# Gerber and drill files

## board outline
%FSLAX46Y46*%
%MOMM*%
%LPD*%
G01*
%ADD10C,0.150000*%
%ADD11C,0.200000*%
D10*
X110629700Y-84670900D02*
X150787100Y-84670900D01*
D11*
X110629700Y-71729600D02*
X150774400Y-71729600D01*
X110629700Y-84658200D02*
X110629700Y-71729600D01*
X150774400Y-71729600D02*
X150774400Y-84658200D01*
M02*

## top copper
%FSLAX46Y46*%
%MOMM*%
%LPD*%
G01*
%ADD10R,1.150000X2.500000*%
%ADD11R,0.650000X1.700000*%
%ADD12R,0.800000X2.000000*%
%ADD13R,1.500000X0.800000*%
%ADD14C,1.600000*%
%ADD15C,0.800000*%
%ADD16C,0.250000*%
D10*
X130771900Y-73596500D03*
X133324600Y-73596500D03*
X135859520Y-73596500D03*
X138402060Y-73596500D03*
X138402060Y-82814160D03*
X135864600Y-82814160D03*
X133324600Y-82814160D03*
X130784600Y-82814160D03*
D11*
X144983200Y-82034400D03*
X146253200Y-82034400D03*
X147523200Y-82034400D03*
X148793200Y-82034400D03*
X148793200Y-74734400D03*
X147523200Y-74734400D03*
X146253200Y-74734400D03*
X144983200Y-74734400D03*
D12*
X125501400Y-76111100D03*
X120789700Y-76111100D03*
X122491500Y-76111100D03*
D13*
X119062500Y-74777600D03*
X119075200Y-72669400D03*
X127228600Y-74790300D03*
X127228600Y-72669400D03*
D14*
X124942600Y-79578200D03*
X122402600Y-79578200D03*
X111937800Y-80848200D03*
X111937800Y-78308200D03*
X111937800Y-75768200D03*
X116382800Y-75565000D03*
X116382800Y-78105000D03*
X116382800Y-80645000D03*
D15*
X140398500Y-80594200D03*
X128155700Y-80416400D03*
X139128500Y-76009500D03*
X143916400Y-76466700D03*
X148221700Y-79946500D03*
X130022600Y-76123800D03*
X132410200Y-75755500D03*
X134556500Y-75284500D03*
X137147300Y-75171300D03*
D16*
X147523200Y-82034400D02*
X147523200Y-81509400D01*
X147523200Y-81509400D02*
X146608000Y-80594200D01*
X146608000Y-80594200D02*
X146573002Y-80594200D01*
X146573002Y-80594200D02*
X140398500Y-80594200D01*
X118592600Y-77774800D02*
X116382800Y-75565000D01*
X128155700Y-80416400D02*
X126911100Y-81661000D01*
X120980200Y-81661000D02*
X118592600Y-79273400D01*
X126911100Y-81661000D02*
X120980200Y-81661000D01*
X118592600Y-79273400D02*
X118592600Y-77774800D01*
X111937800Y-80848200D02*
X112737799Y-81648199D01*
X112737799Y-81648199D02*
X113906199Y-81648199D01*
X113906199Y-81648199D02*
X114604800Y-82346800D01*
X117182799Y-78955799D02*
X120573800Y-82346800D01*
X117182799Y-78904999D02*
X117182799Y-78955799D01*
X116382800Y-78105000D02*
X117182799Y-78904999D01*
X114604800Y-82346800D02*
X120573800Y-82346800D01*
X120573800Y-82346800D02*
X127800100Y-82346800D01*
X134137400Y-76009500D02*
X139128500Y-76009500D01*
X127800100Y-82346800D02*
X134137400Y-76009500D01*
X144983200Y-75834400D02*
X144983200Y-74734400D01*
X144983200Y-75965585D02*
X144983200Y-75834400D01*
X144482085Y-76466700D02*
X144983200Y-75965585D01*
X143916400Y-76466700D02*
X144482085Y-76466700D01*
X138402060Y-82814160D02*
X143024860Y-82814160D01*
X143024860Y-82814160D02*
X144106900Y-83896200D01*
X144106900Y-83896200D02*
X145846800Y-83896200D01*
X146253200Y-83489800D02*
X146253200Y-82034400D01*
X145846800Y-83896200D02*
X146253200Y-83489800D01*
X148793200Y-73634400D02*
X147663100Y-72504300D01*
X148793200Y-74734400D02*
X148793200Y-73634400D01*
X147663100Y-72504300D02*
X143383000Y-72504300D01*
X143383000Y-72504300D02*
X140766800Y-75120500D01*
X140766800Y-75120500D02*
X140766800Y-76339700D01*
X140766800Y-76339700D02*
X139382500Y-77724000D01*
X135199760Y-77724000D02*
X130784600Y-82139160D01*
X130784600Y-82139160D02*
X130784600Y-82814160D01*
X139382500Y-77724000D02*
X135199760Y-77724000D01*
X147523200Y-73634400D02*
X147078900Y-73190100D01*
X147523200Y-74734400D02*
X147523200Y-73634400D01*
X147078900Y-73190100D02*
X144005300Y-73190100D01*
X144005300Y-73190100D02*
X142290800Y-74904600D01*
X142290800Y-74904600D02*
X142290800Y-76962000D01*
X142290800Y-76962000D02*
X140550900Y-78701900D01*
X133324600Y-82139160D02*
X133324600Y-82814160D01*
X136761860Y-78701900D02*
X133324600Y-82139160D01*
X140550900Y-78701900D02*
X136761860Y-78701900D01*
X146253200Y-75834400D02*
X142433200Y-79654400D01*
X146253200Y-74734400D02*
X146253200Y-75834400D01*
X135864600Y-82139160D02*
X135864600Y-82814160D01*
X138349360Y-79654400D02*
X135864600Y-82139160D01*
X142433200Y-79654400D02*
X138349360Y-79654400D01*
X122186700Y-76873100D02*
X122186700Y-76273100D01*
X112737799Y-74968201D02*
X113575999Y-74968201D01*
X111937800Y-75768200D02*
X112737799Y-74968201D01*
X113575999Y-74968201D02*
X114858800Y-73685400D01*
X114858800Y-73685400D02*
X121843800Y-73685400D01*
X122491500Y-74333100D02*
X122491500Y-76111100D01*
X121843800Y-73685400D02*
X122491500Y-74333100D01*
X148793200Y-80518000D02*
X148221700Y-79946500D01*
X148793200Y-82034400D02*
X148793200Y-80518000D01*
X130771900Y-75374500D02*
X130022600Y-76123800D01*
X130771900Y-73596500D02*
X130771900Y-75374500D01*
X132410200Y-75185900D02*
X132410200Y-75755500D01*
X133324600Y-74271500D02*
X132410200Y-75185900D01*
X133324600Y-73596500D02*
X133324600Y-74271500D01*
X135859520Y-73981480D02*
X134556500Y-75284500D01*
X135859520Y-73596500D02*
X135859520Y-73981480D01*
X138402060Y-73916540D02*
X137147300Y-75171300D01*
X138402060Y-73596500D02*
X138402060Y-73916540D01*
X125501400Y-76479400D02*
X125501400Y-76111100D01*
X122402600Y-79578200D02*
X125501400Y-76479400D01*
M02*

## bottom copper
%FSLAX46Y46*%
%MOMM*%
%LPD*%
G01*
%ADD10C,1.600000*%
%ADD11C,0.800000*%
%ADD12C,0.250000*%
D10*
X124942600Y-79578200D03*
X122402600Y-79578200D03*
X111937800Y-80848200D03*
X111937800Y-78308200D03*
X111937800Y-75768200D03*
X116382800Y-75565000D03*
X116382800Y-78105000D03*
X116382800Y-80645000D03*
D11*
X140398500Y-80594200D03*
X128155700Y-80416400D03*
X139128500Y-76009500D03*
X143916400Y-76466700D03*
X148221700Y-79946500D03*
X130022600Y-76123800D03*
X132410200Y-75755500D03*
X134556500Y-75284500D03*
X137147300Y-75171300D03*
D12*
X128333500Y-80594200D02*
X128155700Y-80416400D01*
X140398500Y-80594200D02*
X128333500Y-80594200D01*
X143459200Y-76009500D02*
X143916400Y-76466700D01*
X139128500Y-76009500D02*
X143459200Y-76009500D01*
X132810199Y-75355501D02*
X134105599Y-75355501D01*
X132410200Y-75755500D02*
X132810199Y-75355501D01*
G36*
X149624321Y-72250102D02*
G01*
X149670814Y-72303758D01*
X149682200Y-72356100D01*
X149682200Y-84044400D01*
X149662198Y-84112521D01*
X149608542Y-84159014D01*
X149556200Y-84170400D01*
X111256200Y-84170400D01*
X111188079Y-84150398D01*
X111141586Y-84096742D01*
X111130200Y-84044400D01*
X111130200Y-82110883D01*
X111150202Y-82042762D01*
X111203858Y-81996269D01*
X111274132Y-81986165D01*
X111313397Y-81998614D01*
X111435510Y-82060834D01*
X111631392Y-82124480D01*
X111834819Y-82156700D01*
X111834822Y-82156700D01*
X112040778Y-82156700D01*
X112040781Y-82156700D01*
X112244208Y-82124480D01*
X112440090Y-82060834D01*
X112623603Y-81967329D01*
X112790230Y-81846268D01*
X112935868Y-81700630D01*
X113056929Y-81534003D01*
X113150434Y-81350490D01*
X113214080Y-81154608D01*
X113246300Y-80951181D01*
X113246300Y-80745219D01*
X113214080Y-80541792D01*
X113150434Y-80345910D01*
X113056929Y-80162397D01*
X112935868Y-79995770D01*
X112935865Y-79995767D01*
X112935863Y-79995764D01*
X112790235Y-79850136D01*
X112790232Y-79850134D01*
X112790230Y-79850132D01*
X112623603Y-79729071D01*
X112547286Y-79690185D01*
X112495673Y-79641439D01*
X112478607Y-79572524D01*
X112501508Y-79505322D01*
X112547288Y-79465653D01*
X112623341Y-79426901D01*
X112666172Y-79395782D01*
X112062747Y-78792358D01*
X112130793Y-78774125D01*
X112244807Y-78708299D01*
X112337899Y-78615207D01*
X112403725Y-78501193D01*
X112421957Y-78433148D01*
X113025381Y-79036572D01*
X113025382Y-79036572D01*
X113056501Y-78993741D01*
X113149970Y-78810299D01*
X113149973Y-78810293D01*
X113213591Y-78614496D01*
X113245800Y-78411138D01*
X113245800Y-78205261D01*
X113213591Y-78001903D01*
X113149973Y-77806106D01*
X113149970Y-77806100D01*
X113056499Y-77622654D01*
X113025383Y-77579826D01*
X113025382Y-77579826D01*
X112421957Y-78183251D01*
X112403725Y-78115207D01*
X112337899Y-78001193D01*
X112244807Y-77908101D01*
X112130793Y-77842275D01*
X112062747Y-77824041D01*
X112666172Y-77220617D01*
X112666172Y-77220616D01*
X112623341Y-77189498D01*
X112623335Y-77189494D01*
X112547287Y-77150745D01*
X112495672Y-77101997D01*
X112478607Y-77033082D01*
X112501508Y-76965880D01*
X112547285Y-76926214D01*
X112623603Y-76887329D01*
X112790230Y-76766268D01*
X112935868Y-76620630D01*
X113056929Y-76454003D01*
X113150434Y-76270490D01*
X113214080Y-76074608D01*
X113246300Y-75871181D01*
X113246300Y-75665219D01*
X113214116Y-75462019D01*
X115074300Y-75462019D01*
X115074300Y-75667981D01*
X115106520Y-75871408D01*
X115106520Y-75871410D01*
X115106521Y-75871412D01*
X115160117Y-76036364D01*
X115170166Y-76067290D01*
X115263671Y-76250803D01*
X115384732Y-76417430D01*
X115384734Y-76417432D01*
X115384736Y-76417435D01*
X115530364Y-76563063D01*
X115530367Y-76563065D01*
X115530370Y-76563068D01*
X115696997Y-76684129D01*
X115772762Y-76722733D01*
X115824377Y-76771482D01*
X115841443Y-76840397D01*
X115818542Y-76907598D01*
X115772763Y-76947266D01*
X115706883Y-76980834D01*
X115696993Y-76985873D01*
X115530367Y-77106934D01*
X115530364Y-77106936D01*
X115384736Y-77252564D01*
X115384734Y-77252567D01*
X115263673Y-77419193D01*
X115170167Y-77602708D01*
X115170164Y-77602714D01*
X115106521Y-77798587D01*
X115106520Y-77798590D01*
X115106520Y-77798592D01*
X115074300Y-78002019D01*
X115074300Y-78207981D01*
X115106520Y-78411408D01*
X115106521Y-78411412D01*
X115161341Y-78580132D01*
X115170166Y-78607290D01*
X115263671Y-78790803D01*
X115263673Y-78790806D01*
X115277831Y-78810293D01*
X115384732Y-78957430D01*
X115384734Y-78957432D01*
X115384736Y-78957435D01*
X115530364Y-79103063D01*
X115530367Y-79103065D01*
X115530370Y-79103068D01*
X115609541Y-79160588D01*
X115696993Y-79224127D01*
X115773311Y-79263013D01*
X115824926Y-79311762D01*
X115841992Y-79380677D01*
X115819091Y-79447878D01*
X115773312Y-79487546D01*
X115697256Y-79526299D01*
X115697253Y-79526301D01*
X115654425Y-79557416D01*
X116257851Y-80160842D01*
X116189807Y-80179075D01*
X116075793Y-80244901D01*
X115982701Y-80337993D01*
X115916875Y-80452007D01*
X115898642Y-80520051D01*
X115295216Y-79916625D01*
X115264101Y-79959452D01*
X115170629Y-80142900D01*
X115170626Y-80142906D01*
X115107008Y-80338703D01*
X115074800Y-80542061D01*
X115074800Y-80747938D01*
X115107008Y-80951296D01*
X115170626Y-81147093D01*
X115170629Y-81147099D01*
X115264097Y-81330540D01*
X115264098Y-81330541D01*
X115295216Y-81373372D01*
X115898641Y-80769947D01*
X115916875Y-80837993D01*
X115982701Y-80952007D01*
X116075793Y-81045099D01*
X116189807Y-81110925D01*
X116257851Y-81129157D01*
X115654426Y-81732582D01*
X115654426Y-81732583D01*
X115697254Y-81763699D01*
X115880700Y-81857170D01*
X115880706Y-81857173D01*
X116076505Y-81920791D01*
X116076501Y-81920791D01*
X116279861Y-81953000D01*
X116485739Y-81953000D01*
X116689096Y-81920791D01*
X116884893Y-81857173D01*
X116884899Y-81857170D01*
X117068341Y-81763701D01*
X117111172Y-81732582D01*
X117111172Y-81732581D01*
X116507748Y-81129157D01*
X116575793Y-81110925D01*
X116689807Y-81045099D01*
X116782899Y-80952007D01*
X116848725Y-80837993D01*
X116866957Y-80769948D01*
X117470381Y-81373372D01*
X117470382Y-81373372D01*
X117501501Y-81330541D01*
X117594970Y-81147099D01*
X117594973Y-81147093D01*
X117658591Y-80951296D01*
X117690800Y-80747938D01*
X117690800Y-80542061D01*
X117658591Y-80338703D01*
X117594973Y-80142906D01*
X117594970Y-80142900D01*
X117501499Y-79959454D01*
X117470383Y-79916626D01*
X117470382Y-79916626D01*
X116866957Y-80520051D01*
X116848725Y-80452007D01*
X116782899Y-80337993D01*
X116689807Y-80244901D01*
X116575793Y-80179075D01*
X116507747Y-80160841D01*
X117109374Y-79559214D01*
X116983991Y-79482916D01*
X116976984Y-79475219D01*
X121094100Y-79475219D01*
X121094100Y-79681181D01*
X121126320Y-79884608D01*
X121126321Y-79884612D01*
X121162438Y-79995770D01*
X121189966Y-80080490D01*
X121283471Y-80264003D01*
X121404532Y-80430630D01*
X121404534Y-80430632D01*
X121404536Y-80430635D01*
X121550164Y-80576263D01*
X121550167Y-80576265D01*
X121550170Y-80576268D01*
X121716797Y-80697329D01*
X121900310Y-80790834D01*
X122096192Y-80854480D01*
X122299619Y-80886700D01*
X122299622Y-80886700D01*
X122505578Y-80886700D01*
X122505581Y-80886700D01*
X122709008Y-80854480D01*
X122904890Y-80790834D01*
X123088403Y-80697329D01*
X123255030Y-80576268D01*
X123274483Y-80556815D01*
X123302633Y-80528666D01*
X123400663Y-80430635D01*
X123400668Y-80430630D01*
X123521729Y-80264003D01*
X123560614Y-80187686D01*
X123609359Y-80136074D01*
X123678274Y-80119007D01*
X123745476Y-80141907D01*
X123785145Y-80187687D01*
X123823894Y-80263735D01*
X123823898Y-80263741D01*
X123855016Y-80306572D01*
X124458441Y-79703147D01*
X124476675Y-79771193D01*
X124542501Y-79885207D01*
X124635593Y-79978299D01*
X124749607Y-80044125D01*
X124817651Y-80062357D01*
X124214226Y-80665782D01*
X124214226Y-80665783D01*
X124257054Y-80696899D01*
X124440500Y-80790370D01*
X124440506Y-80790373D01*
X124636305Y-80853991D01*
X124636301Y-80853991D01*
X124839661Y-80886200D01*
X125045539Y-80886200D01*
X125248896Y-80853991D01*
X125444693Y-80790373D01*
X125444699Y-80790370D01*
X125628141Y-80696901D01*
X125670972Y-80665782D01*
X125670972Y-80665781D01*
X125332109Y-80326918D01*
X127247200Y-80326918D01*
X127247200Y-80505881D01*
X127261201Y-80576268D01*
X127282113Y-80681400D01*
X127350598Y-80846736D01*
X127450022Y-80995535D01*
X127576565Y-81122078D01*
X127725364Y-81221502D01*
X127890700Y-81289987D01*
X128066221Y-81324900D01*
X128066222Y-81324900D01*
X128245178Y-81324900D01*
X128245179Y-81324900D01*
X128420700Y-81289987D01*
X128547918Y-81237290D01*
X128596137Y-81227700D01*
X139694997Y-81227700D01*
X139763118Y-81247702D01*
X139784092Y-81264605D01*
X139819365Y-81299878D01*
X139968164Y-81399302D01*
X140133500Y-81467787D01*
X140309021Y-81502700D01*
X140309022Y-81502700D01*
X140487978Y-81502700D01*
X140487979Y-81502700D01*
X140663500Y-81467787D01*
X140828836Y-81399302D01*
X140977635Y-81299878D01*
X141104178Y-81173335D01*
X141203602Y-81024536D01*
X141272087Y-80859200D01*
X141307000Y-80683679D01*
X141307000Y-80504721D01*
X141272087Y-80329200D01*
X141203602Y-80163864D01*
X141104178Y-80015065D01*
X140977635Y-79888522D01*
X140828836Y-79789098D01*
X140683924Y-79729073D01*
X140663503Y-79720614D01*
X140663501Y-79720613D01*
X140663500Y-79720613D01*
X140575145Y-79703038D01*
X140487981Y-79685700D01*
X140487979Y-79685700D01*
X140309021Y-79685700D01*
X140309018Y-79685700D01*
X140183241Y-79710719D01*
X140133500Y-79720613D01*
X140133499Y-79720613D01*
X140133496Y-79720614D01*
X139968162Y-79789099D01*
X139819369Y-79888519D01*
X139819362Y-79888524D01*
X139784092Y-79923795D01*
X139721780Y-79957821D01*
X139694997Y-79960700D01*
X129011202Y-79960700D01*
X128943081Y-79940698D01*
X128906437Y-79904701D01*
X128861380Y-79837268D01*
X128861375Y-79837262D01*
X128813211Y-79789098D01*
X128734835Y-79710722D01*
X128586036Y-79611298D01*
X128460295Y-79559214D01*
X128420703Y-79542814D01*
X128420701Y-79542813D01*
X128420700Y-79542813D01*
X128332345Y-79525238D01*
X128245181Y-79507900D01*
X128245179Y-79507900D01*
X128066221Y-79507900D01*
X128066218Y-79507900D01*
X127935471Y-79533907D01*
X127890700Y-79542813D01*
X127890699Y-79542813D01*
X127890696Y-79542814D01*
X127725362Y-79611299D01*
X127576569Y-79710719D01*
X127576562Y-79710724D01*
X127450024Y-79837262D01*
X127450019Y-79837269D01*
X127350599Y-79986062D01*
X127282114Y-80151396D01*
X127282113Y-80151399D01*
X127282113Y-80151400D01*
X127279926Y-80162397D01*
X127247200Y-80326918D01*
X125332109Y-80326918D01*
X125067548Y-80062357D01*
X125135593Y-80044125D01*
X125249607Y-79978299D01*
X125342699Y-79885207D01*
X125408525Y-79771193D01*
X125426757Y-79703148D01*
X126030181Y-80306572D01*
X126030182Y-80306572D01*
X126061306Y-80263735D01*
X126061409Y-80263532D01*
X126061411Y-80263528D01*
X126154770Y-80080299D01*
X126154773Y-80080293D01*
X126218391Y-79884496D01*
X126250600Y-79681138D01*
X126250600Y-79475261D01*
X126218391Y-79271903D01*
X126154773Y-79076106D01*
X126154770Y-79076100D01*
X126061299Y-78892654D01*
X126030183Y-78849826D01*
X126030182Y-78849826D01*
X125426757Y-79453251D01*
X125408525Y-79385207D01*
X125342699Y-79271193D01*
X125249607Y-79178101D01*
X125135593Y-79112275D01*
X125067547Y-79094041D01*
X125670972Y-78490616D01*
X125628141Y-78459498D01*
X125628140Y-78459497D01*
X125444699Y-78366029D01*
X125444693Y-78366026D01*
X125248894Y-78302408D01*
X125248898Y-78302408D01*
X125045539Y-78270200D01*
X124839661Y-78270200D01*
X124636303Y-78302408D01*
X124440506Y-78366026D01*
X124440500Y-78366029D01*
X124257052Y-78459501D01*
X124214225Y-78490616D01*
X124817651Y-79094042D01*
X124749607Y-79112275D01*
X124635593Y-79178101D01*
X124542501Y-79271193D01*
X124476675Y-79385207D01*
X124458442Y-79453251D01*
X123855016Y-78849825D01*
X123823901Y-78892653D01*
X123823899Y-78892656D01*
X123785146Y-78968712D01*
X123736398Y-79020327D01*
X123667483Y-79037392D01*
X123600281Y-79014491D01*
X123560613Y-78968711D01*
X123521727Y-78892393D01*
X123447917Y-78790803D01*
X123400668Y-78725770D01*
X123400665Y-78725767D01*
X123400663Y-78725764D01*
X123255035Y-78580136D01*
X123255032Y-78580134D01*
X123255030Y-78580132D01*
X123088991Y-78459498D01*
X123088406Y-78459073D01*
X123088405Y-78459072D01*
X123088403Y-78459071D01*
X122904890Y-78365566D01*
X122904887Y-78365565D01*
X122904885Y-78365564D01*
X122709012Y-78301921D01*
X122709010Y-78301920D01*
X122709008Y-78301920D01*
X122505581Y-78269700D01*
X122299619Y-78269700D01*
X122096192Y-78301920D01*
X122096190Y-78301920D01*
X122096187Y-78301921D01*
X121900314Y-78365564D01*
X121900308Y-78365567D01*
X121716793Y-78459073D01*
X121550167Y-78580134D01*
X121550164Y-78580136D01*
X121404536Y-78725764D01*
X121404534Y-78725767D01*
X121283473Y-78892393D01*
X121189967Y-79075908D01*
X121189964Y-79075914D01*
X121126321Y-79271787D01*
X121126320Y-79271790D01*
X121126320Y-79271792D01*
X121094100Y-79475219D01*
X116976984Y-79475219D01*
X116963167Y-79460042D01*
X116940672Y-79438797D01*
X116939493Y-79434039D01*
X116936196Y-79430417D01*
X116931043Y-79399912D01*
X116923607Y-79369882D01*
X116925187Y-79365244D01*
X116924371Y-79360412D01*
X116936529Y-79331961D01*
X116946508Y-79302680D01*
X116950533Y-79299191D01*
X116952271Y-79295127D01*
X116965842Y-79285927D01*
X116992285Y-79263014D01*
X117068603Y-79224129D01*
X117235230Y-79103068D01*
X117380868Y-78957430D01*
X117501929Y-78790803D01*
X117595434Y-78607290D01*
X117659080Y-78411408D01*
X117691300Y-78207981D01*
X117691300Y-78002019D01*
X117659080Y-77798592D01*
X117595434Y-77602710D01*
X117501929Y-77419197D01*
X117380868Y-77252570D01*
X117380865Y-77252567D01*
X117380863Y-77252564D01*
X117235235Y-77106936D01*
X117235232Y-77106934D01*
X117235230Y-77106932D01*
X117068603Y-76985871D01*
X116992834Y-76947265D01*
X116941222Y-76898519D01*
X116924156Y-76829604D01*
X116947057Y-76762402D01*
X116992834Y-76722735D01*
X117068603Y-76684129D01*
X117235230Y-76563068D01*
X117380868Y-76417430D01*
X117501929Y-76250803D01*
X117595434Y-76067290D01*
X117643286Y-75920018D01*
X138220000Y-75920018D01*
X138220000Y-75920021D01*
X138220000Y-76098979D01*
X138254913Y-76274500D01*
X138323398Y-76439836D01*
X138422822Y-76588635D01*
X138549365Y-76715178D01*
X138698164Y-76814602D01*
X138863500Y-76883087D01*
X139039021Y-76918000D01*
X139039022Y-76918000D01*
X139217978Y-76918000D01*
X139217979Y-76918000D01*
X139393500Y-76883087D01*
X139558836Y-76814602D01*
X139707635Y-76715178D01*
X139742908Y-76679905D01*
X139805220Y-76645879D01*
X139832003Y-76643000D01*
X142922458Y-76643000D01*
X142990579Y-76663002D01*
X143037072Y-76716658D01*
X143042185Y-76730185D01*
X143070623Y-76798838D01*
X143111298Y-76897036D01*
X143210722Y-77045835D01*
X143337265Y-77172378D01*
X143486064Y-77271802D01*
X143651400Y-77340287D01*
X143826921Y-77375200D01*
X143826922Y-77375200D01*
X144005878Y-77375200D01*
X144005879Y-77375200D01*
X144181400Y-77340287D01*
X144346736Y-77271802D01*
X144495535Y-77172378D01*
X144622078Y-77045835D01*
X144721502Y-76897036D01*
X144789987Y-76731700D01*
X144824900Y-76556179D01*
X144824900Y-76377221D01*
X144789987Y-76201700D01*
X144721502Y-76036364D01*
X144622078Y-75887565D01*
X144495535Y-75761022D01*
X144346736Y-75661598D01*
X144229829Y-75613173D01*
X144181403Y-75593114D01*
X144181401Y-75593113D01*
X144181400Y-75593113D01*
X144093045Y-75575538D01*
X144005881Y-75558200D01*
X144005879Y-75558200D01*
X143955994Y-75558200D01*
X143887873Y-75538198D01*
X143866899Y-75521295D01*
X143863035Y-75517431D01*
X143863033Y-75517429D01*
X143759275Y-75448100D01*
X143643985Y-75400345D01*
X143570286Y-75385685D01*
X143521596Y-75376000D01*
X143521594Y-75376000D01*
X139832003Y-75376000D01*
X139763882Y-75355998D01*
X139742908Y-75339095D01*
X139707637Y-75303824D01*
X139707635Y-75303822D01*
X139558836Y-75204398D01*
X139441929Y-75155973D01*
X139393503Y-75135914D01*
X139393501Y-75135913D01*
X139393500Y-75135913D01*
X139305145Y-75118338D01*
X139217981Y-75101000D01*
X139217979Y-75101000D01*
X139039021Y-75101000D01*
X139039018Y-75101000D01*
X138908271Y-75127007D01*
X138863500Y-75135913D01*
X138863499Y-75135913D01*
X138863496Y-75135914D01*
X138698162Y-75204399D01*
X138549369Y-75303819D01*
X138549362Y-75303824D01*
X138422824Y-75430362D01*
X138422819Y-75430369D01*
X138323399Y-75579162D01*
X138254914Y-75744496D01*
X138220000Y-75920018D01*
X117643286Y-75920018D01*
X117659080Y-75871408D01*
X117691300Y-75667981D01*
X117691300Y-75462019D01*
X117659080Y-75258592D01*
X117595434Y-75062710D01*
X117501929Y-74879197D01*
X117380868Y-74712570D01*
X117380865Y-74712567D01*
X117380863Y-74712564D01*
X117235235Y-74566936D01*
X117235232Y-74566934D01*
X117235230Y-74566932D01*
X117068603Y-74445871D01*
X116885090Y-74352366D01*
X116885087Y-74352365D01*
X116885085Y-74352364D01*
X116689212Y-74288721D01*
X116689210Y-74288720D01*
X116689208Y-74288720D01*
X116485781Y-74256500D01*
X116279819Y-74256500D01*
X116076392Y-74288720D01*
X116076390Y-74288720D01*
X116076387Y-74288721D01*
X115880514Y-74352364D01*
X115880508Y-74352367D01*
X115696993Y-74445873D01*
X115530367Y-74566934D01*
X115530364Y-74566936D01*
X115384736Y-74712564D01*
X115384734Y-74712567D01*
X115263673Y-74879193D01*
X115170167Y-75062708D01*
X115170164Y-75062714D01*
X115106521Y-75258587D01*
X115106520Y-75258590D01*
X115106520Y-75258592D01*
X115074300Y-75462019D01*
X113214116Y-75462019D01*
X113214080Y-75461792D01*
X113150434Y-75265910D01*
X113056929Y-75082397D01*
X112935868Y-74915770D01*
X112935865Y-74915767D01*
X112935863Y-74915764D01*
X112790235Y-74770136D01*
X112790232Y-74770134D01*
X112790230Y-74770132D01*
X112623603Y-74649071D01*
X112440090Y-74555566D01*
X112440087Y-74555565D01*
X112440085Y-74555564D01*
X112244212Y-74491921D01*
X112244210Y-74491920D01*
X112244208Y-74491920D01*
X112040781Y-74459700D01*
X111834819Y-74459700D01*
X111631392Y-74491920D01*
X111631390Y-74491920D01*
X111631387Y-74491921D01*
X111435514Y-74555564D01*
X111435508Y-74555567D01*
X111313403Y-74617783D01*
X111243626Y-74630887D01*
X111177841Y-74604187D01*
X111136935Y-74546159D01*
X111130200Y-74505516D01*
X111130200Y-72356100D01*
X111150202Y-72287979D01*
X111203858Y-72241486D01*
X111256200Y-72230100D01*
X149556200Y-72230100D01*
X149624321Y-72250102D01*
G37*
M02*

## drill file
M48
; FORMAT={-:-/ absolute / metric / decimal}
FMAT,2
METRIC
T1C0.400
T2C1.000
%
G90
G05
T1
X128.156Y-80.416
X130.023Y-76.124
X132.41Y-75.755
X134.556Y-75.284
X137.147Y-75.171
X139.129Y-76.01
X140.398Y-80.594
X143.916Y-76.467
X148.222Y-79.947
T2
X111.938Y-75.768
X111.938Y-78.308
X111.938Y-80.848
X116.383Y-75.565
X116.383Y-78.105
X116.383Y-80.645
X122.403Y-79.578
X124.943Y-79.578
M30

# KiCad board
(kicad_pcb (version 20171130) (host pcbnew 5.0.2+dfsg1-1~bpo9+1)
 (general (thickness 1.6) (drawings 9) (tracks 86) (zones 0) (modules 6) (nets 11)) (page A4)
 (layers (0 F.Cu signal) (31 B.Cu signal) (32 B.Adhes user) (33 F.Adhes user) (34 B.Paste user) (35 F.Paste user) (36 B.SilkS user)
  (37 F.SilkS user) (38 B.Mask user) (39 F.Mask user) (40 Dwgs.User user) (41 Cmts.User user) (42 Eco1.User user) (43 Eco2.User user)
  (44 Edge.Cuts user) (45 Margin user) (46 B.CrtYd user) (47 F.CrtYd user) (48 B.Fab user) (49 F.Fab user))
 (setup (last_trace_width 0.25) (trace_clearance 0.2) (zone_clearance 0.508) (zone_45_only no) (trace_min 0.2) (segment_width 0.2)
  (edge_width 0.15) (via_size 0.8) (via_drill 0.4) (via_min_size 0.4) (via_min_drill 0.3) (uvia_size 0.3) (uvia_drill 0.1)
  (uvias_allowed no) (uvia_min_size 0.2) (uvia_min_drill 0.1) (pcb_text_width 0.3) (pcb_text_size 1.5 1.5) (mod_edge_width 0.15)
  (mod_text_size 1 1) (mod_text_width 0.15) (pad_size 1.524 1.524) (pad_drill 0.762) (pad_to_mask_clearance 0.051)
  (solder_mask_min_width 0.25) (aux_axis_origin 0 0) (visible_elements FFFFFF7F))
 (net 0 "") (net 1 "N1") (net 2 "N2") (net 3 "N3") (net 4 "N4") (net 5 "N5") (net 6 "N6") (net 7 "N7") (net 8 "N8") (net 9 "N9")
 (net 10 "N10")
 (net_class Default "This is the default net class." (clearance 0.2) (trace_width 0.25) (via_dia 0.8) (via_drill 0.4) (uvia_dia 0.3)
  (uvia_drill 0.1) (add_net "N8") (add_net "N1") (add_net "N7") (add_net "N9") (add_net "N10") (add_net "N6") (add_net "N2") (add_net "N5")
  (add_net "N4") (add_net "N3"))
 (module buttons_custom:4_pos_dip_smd (layer F.Cu) (at 134.5946 78.2066)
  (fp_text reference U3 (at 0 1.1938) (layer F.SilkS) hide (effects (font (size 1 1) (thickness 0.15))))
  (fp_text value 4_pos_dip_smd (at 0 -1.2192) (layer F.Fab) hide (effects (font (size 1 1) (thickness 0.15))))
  (pad 1 smd rect (at -3.8227 -4.6101) (size 1.15 2.5) (layers F.Cu F.Paste F.Mask) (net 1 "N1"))
  (pad 2 smd rect (at -1.27 -4.6101) (size 1.15 2.5) (layers F.Cu F.Paste F.Mask) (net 1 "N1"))
  (pad 3 smd rect (at 1.26492 -4.6101) (size 1.15 2.5) (layers F.Cu F.Paste F.Mask) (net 1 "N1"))
  (pad 4 smd rect (at 3.80746 -4.6101) (size 1.15 2.5) (layers F.Cu F.Paste F.Mask) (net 1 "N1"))
  (pad 5 smd rect (at 3.80746 4.60756) (size 1.15 2.5) (layers F.Cu F.Paste F.Mask) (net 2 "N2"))
  (pad 6 smd rect (at 1.27 4.60756) (size 1.15 2.5) (layers F.Cu F.Paste F.Mask) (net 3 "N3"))
  (pad 7 smd rect (at -1.27 4.60756) (size 1.15 2.5) (layers F.Cu F.Paste F.Mask) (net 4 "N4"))
  (pad 8 smd rect (at -3.81 4.60756) (size 1.15 2.5) (layers F.Cu F.Paste F.Mask) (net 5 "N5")))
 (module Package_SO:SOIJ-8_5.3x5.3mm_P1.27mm (layer F.Cu) (at 146.8882 78.3844 90)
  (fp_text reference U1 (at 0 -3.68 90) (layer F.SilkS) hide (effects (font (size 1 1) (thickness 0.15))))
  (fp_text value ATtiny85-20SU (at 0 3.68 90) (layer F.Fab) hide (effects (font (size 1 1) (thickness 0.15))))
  (pad 1 smd rect (at -3.65 -1.905 90) (size 1.7 0.65) (layers F.Cu F.Paste F.Mask) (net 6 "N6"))
  (pad 2 smd rect (at -3.65 -0.635 90) (size 1.7 0.65) (layers F.Cu F.Paste F.Mask) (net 2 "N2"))
  (pad 3 smd rect (at -3.65 0.635 90) (size 1.7 0.65) (layers F.Cu F.Paste F.Mask) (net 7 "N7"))
  (pad 4 smd rect (at -3.65 1.905 90) (size 1.7 0.65) (layers F.Cu F.Paste F.Mask) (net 1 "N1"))
  (pad 5 smd rect (at 3.65 1.905 90) (size 1.7 0.65) (layers F.Cu F.Paste F.Mask) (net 5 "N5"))
  (pad 6 smd rect (at 3.65 0.635 90) (size 1.7 0.65) (layers F.Cu F.Paste F.Mask) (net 4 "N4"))
  (pad 7 smd rect (at 3.65 -0.635 90) (size 1.7 0.65) (layers F.Cu F.Paste F.Mask) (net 3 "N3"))
  (pad 8 smd rect (at 3.65 -1.905 90) (size 1.7 0.65) (layers F.Cu F.Paste F.Mask) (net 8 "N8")))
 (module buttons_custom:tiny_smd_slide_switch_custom (layer F.Cu) (at 125.5014 75.1078 180)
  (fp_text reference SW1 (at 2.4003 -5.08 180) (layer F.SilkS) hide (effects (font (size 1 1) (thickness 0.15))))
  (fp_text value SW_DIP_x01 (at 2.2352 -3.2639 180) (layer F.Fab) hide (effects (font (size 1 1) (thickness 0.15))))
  (pad 1 smd rect (at 0 -1.0033 180) (size 0.8 2) (layers F.Cu F.Paste F.Mask) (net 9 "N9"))
  (pad 3 smd rect (at 4.7117 -1.0033 180) (size 0.8 2) (layers F.Cu F.Paste F.Mask))
  (pad 2 smd rect (at 3.0099 -1.0033 180) (size 0.8 2) (layers F.Cu F.Paste F.Mask) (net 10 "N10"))
  (pad 4 smd rect (at 6.4389 0.3302 270) (size 0.8 1.5) (layers F.Cu F.Paste F.Mask))
  (pad 4 smd rect (at 6.4262 2.4384 270) (size 0.8 1.5) (layers F.Cu F.Paste F.Mask))
  (pad 4 smd rect (at -1.7272 0.3175 270) (size 0.8 1.5) (layers F.Cu F.Paste F.Mask))
  (pad 4 smd rect (at -1.7272 2.4384 270) (size 0.8 1.5) (layers F.Cu F.Paste F.Mask)))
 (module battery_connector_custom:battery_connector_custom (layer F.Cu) (at 123.6726 79.5782 180)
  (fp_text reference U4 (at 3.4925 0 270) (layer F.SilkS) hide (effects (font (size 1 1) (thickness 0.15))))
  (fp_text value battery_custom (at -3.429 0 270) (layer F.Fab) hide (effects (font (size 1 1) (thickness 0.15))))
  (pad 1 thru_hole circle (at -1.27 0 180) (size 1.6 1.6) (drill 1) (layers *.Cu *.Mask) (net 1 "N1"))
  (pad 2 thru_hole circle (at 1.27 0 180) (size 1.6 1.6) (drill 1) (layers *.Cu *.Mask) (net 9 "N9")))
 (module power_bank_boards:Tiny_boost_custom (layer B.Cu) (at 108.5596 78.105 180)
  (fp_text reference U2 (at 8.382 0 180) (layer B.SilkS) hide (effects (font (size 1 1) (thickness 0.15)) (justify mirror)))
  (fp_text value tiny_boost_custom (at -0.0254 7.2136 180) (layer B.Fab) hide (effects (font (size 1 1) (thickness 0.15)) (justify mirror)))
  (pad 3 thru_hole circle (at -3.3782 -2.7432 180) (size 1.6 1.6) (drill 1) (layers *.Cu *.Mask) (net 8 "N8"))
  (pad 2 thru_hole circle (at -3.3782 -0.2032 180) (size 1.6 1.6) (drill 1) (layers *.Cu *.Mask) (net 1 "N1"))
  (pad 1 thru_hole circle (at -3.3782 2.3368 180) (size 1.6 1.6) (drill 1) (layers *.Cu *.Mask) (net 10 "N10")))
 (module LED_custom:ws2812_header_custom (layer F.Cu) (at 116.3828 78.105 270)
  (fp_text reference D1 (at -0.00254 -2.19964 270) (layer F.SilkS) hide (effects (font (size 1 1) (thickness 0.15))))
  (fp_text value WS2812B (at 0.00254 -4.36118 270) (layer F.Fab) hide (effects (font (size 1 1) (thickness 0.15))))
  (pad 4 thru_hole circle (at -2.54 0 270) (size 1.6 1.6) (drill 1) (layers *.Cu *.Mask) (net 7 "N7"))
  (pad 1 thru_hole circle (at 0 0 270) (size 1.6 1.6) (drill 1) (layers *.Cu *.Mask) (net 8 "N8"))
  (pad 3 thru_hole circle (at 2.54 0 270) (size 1.6 1.6) (drill 1) (layers *.Cu *.Mask) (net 1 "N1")))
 (gr_line (start 110.6297 84.6709) (end 150.7871 84.6709) (layer Edge.Cuts) (width 0.15))
 (gr_line (start 110.6297 71.7296) (end 150.7744 71.7296) (layer Edge.Cuts) (width 0.2))
 (gr_line (start 110.6297 84.6582) (end 110.6297 71.7296) (layer Edge.Cuts) (width 0.2))
 (gr_line (start 150.7744 71.7296) (end 150.7744 84.6582) (layer Edge.Cuts) (width 0.2))
 (via (at 140.3985 80.5942) (size 0.8) (drill 0.4) (layers F.Cu B.Cu) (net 7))
 (segment (start 147.5232 82.0344) (end 147.5232 81.5094) (width 0.25) (layer F.Cu) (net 7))
 (segment (start 147.5232 81.5094) (end 146.608 80.5942) (width 0.25) (layer F.Cu) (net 7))
 (segment (start 146.608 80.5942) (end 146.573002 80.5942) (width 0.25) (layer F.Cu) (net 7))
 (segment (start 146.573002 80.5942) (end 140.3985 80.5942) (width 0.25) (layer F.Cu) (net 7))
 (via (at 128.1557 80.4164) (size 0.8) (drill 0.4) (layers F.Cu B.Cu) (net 7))
 (segment (start 128.3335 80.5942) (end 128.1557 80.4164) (width 0.25) (layer B.Cu) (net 7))
 (segment (start 140.3985 80.5942) (end 128.3335 80.5942) (width 0.25) (layer B.Cu) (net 7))
 (segment (start 118.5926 77.7748) (end 116.3828 75.565) (width 0.25) (layer F.Cu) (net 7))
 (segment (start 128.1557 80.4164) (end 126.9111 81.661) (width 0.25) (layer F.Cu) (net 7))
 (segment (start 120.9802 81.661) (end 118.5926 79.2734) (width 0.25) (layer F.Cu) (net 7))
 (segment (start 126.9111 81.661) (end 120.9802 81.661) (width 0.25) (layer F.Cu) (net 7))
 (segment (start 118.5926 79.2734) (end 118.5926 77.7748) (width 0.25) (layer F.Cu) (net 7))
 (segment (start 111.9378 80.8482) (end 112.737799 81.648199) (width 0.25) (layer F.Cu) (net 8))
 (segment (start 112.737799 81.648199) (end 113.906199 81.648199) (width 0.25) (layer F.Cu) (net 8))
 (segment (start 113.906199 81.648199) (end 114.6048 82.3468) (width 0.25) (layer F.Cu) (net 8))
 (segment (start 117.182799 78.955799) (end 120.5738 82.3468) (width 0.25) (layer F.Cu) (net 8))
 (segment (start 117.182799 78.904999) (end 117.182799 78.955799) (width 0.25) (layer F.Cu) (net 8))
 (segment (start 116.3828 78.105) (end 117.182799 78.904999) (width 0.25) (layer F.Cu) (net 8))
 (segment (start 114.6048 82.3468) (end 120.5738 82.3468) (width 0.25) (layer F.Cu) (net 8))
 (segment (start 120.5738 82.3468) (end 127.8001 82.3468) (width 0.25) (layer F.Cu) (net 8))
 (via (at 139.1285 76.0095) (size 0.8) (drill 0.4) (layers F.Cu B.Cu) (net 8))
 (segment (start 134.1374 76.0095) (end 139.1285 76.0095) (width 0.25) (layer F.Cu) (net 8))
 (segment (start 127.8001 82.3468) (end 134.1374 76.0095) (width 0.25) (layer F.Cu) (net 8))
 (via (at 143.9164 76.4667) (size 0.8) (drill 0.4) (layers F.Cu B.Cu) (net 8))
 (segment (start 143.4592 76.0095) (end 143.9164 76.4667) (width 0.25) (layer B.Cu) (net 8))
 (segment (start 139.1285 76.0095) (end 143.4592 76.0095) (width 0.25) (layer B.Cu) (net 8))
 (segment (start 144.9832 75.8344) (end 144.9832 74.7344) (width 0.25) (layer F.Cu) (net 8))
 (segment (start 144.9832 75.965585) (end 144.9832 75.8344) (width 0.25) (layer F.Cu) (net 8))
 (segment (start 144.482085 76.4667) (end 144.9832 75.965585) (width 0.25) (layer F.Cu) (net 8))
 (segment (start 143.9164 76.4667) (end 144.482085 76.4667) (width 0.25) (layer F.Cu) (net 8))
 (segment (start 138.40206 82.81416) (end 143.02486 82.81416) (width 0.25) (layer F.Cu) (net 2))
 (segment (start 143.02486 82.81416) (end 144.1069 83.8962) (width 0.25) (layer F.Cu) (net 2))
 (segment (start 144.1069 83.8962) (end 145.8468 83.8962) (width 0.25) (layer F.Cu) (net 2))
 (segment (start 146.2532 83.4898) (end 146.2532 82.0344) (width 0.25) (layer F.Cu) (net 2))
 (segment (start 145.8468 83.8962) (end 146.2532 83.4898) (width 0.25) (layer F.Cu) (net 2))
 (segment (start 148.7932 73.6344) (end 147.6631 72.5043) (width 0.25) (layer F.Cu) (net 5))
 (segment (start 148.7932 74.7344) (end 148.7932 73.6344) (width 0.25) (layer F.Cu) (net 5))
 (segment (start 147.6631 72.5043) (end 143.383 72.5043) (width 0.25) (layer F.Cu) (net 5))
 (segment (start 143.383 72.5043) (end 140.7668 75.1205) (width 0.25) (layer F.Cu) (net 5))
 (segment (start 140.7668 75.1205) (end 140.7668 76.3397) (width 0.25) (layer F.Cu) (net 5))
 (segment (start 140.7668 76.3397) (end 139.3825 77.724) (width 0.25) (layer F.Cu) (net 5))
 (segment (start 135.19976 77.724) (end 130.7846 82.13916) (width 0.25) (layer F.Cu) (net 5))
 (segment (start 130.7846 82.13916) (end 130.7846 82.81416) (width 0.25) (layer F.Cu) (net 5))
 (segment (start 139.3825 77.724) (end 135.19976 77.724) (width 0.25) (layer F.Cu) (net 5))
 (segment (start 147.5232 73.6344) (end 147.0789 73.1901) (width 0.25) (layer F.Cu) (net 4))
 (segment (start 147.5232 74.7344) (end 147.5232 73.6344) (width 0.25) (layer F.Cu) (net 4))
 (segment (start 147.0789 73.1901) (end 144.0053 73.1901) (width 0.25) (layer F.Cu) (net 4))
 (segment (start 144.0053 73.1901) (end 142.2908 74.9046) (width 0.25) (layer F.Cu) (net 4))
 (segment (start 142.2908 74.9046) (end 142.2908 76.962) (width 0.25) (layer F.Cu) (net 4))
 (segment (start 142.2908 76.962) (end 140.5509 78.7019) (width 0.25) (layer F.Cu) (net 4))
 (segment (start 133.3246 82.13916) (end 133.3246 82.81416) (width 0.25) (layer F.Cu) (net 4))
 (segment (start 136.76186 78.7019) (end 133.3246 82.13916) (width 0.25) (layer F.Cu) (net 4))
 (segment (start 140.5509 78.7019) (end 136.76186 78.7019) (width 0.25) (layer F.Cu) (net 4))
 (segment (start 146.2532 75.8344) (end 142.4332 79.6544) (width 0.25) (layer F.Cu) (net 3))
 (segment (start 146.2532 74.7344) (end 146.2532 75.8344) (width 0.25) (layer F.Cu) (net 3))
 (segment (start 135.8646 82.13916) (end 135.8646 82.81416) (width 0.25) (layer F.Cu) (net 3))
 (segment (start 138.34936 79.6544) (end 135.8646 82.13916) (width 0.25) (layer F.Cu) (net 3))
 (segment (start 142.4332 79.6544) (end 138.34936 79.6544) (width 0.25) (layer F.Cu) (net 3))
 (segment (start 122.1867 76.8731) (end 122.1867 76.2731) (width 0.25) (layer F.Cu) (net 10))
 (segment (start 112.737799 74.968201) (end 113.575999 74.968201) (width 0.25) (layer F.Cu) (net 10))
 (segment (start 111.9378 75.7682) (end 112.737799 74.968201) (width 0.25) (layer F.Cu) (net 10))
 (segment (start 113.575999 74.968201) (end 114.8588 73.6854) (width 0.25) (layer F.Cu) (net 10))
 (segment (start 114.8588 73.6854) (end 121.8438 73.6854) (width 0.25) (layer F.Cu) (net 10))
 (segment (start 122.4915 74.3331) (end 122.4915 76.1111) (width 0.25) (layer F.Cu) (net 10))
 (segment (start 121.8438 73.6854) (end 122.4915 74.3331) (width 0.25) (layer F.Cu) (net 10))
 (via (at 148.2217 79.9465) (size 0.8) (drill 0.4) (layers F.Cu B.Cu) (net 1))
 (segment (start 148.7932 80.518) (end 148.2217 79.9465) (width 0.25) (layer F.Cu) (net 1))
 (segment (start 148.7932 82.0344) (end 148.7932 80.518) (width 0.25) (layer F.Cu) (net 1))
 (via (at 130.0226 76.1238) (size 0.8) (drill 0.4) (layers F.Cu B.Cu) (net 1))
 (segment (start 130.7719 75.3745) (end 130.0226 76.1238) (width 0.25) (layer F.Cu) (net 1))
 (segment (start 130.7719 73.5965) (end 130.7719 75.3745) (width 0.25) (layer F.Cu) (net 1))
 (segment (start 132.4102 75.1859) (end 132.4102 75.7555) (width 0.25) (layer F.Cu) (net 1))
 (segment (start 133.3246 74.2715) (end 132.4102 75.1859) (width 0.25) (layer F.Cu) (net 1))
 (via (at 132.4102 75.7555) (size 0.8) (drill 0.4) (layers F.Cu B.Cu) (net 1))
 (segment (start 133.3246 73.5965) (end 133.3246 74.2715) (width 0.25) (layer F.Cu) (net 1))
 (segment (start 132.810199 75.355501) (end 134.105599 75.355501) (width 0.25) (layer B.Cu) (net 1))
 (segment (start 132.4102 75.7555) (end 132.810199 75.355501) (width 0.25) (layer B.Cu) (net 1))
 (segment (start 135.85952 73.98148) (end 134.5565 75.2845) (width 0.25) (layer F.Cu) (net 1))
 (via (at 134.5565 75.2845) (size 0.8) (drill 0.4) (layers F.Cu B.Cu) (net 1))
 (segment (start 135.85952 73.5965) (end 135.85952 73.98148) (width 0.25) (layer F.Cu) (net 1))
 (via (at 137.1473 75.1713) (size 0.8) (drill 0.4) (layers F.Cu B.Cu) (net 1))
 (segment (start 138.40206 73.91654) (end 137.1473 75.1713) (width 0.25) (layer F.Cu) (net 1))
 (segment (start 138.40206 73.5965) (end 138.40206 73.91654) (width 0.25) (layer F.Cu) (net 1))
 (segment (start 125.5014 76.4794) (end 125.5014 76.1111) (width 0.25) (layer F.Cu) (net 9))
 (segment (start 122.4026 79.5782) (end 125.5014 76.4794) (width 0.25) (layer F.Cu) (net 9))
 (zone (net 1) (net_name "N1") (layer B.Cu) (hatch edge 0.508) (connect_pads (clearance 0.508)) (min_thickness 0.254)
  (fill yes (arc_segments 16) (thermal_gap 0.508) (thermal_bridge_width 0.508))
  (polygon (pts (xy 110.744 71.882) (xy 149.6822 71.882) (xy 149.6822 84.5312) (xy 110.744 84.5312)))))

